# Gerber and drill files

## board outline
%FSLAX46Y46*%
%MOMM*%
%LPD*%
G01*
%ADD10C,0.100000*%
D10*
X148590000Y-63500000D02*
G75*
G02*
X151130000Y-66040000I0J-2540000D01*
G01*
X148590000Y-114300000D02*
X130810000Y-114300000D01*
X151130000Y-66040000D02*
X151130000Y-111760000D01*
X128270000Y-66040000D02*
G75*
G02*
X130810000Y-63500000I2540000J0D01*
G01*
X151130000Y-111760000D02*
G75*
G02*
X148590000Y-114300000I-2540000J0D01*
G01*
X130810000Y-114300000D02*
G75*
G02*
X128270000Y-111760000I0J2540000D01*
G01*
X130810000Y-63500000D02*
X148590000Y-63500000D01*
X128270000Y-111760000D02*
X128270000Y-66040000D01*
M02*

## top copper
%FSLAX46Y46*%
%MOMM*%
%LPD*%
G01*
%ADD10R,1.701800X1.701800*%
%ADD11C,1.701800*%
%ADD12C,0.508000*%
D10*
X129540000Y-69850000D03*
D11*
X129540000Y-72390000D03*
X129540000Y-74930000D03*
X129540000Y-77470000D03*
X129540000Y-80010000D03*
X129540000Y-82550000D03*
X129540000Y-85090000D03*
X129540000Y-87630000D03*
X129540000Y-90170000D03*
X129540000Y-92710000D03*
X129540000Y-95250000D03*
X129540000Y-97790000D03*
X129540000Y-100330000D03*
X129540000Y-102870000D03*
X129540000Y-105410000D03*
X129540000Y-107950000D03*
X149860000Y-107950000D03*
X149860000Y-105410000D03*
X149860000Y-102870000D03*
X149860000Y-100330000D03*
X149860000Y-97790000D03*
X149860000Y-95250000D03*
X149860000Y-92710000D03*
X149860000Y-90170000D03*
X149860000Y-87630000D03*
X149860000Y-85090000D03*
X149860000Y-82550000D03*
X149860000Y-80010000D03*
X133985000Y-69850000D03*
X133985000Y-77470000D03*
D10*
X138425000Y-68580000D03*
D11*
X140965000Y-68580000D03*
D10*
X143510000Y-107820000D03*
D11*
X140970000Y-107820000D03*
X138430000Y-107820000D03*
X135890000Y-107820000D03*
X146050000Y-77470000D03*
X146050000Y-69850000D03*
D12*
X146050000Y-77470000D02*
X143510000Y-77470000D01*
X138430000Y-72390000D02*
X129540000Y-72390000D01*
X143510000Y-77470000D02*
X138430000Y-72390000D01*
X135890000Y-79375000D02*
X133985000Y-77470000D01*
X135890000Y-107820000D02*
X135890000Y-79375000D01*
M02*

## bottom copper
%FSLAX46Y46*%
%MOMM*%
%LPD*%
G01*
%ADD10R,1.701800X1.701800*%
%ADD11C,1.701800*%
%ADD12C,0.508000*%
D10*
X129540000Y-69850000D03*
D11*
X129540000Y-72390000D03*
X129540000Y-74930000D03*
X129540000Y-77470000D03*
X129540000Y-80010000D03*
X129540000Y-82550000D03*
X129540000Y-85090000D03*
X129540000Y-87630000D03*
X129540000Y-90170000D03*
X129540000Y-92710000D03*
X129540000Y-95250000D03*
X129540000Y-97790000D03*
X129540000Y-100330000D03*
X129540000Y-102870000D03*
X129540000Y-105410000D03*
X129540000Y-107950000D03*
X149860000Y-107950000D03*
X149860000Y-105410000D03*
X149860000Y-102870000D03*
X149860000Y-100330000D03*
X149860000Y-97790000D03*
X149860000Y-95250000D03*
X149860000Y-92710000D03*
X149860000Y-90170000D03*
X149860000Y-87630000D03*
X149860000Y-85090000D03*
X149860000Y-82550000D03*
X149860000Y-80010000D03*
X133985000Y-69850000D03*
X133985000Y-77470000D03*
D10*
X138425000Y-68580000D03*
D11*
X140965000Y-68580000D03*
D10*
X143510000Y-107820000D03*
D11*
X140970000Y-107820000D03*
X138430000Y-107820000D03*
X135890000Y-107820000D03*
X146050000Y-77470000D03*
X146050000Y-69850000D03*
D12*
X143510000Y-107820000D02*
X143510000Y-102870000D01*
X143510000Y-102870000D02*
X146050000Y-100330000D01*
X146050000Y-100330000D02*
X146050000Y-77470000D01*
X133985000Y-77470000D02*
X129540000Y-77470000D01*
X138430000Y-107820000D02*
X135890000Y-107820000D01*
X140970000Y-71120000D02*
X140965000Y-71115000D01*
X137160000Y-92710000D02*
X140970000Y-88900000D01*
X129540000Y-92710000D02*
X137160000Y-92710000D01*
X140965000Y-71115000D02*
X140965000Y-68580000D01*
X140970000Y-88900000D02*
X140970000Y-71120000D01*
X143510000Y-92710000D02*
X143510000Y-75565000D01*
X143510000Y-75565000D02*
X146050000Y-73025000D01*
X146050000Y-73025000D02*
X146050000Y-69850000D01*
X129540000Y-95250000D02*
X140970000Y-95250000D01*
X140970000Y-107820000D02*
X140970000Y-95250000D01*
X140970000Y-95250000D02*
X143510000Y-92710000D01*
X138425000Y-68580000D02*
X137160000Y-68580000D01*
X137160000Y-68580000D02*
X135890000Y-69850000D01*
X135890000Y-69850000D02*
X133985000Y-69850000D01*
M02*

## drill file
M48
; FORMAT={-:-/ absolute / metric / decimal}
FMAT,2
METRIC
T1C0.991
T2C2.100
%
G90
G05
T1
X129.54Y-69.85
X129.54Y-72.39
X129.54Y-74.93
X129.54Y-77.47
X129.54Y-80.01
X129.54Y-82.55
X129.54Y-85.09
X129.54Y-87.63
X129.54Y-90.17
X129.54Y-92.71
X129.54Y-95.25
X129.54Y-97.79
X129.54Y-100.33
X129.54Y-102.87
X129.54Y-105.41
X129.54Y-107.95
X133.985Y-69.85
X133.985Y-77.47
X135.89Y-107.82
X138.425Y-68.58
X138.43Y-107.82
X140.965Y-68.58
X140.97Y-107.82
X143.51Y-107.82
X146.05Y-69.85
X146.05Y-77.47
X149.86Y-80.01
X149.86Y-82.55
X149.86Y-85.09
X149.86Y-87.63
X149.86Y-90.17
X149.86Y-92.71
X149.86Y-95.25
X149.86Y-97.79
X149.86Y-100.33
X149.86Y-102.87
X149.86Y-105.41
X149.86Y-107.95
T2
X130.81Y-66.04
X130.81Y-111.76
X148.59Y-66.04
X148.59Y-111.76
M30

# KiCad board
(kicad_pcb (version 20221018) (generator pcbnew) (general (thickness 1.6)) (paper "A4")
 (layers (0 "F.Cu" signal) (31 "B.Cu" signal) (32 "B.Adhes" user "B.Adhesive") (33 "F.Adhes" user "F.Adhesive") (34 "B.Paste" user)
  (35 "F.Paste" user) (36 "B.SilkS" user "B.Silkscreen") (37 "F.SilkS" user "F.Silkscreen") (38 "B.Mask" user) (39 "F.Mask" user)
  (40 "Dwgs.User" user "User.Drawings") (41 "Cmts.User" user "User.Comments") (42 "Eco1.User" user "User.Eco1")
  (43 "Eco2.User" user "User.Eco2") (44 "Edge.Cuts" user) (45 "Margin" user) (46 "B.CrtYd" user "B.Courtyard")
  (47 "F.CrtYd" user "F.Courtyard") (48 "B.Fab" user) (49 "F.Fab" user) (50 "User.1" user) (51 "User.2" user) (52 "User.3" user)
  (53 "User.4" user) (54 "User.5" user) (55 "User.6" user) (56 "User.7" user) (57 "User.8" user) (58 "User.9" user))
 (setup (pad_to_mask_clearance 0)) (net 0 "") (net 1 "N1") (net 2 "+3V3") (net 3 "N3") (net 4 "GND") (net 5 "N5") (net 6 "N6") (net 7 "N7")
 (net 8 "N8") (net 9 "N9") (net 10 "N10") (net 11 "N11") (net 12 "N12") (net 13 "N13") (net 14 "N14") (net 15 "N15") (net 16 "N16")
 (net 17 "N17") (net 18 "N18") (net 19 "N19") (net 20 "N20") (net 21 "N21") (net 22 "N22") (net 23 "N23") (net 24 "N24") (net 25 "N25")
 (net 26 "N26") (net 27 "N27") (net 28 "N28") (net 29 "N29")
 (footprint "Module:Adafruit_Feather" (layer "F.Cu") (at 129.54 69.85)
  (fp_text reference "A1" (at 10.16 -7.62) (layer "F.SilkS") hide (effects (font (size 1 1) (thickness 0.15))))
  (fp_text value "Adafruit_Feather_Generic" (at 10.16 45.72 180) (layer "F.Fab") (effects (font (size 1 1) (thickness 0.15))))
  (pad "1" thru_hole rect (at 0 0 180) (size 1.7018 1.7018) (drill 0.9906) (layers "*.Cu" "*.Mask") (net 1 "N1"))
  (pad "2" thru_hole circle (at 0 2.54 180) (size 1.7018 1.6) (drill 0.9906) (layers "*.Cu" "*.Mask") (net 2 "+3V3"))
  (pad "3" thru_hole circle (at 0 5.08 180) (size 1.7018 1.6) (drill 0.9906) (layers "*.Cu" "*.Mask") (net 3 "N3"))
  (pad "4" thru_hole circle (at 0 7.62 180) (size 1.7018 1.6) (drill 0.9906) (layers "*.Cu" "*.Mask") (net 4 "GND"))
  (pad "5" thru_hole circle (at 0 10.16 180) (size 1.7018 1.6) (drill 0.9906) (layers "*.Cu" "*.Mask") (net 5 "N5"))
  (pad "6" thru_hole circle (at 0 12.7 180) (size 1.7018 1.6) (drill 0.9906) (layers "*.Cu" "*.Mask") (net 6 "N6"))
  (pad "7" thru_hole circle (at 0 15.24 180) (size 1.7018 1.6) (drill 0.9906) (layers "*.Cu" "*.Mask") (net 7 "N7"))
  (pad "8" thru_hole circle (at 0 17.78 180) (size 1.7018 1.6) (drill 0.9906) (layers "*.Cu" "*.Mask") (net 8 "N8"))
  (pad "9" thru_hole circle (at 0 20.32 180) (size 1.7018 1.6) (drill 0.9906) (layers "*.Cu" "*.Mask") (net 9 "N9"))
  (pad "10" thru_hole circle (at 0 22.86 180) (size 1.7018 1.6) (drill 0.9906) (layers "*.Cu" "*.Mask") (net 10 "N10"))
  (pad "11" thru_hole circle (at 0 25.4 180) (size 1.7018 1.6) (drill 0.9906) (layers "*.Cu" "*.Mask") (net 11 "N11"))
  (pad "12" thru_hole circle (at 0 27.94 180) (size 1.7018 1.6) (drill 0.9906) (layers "*.Cu" "*.Mask") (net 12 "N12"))
  (pad "13" thru_hole circle (at 0 30.48 180) (size 1.7018 1.6) (drill 0.9906) (layers "*.Cu" "*.Mask") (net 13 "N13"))
  (pad "14" thru_hole circle (at 0 33.02 180) (size 1.7018 1.6) (drill 0.9906) (layers "*.Cu" "*.Mask") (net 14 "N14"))
  (pad "15" thru_hole circle (at 0 35.56 180) (size 1.7018 1.6) (drill 0.9906) (layers "*.Cu" "*.Mask") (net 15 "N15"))
  (pad "16" thru_hole circle (at 0 38.1 180) (size 1.7018 1.6) (drill 0.9906) (layers "*.Cu" "*.Mask") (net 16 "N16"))
  (pad "17" thru_hole circle (at 20.32 38.1 180) (size 1.7018 1.6) (drill 0.9906) (layers "*.Cu" "*.Mask") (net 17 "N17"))
  (pad "18" thru_hole circle (at 20.32 35.56 180) (size 1.7018 1.6) (drill 0.9906) (layers "*.Cu" "*.Mask") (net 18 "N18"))
  (pad "19" thru_hole circle (at 20.32 33.02 180) (size 1.7018 1.6) (drill 0.9906) (layers "*.Cu" "*.Mask") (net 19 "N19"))
  (pad "20" thru_hole circle (at 20.32 30.48 180) (size 1.7018 1.6) (drill 0.9906) (layers "*.Cu" "*.Mask") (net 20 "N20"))
  (pad "21" thru_hole circle (at 20.32 27.94 180) (size 1.7018 1.6) (drill 0.9906) (layers "*.Cu" "*.Mask") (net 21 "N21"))
  (pad "22" thru_hole circle (at 20.32 25.4 180) (size 1.7018 1.6) (drill 0.9906) (layers "*.Cu" "*.Mask") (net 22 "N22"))
  (pad "23" thru_hole circle (at 20.32 22.86 180) (size 1.7018 1.6) (drill 0.9906) (layers "*.Cu" "*.Mask") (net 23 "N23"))
  (pad "24" thru_hole circle (at 20.32 20.32 180) (size 1.7018 1.6) (drill 0.9906) (layers "*.Cu" "*.Mask") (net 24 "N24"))
  (pad "25" thru_hole circle (at 20.32 17.78 180) (size 1.7018 1.6) (drill 0.9906) (layers "*.Cu" "*.Mask") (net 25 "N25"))
  (pad "26" thru_hole circle (at 20.32 15.24 180) (size 1.7018 1.6) (drill 0.9906) (layers "*.Cu" "*.Mask") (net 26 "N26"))
  (pad "27" thru_hole circle (at 20.32 12.7 180) (size 1.7018 1.6) (drill 0.9906) (layers "*.Cu" "*.Mask") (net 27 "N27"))
  (pad "28" thru_hole circle (at 20.32 10.16 180) (size 1.7018 1.6) (drill 0.9906) (layers "*.Cu" "*.Mask") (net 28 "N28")))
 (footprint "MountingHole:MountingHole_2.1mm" (layer "F.Cu") (at 130.81 111.76)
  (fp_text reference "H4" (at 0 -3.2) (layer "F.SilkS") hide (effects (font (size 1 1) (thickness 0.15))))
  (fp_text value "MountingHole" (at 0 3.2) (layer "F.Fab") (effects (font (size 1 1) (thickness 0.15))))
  (pad "" np_thru_hole circle (at 0 0) (size 2.1 2.1) (drill 2.1) (layers "*.Cu" "*.Mask")))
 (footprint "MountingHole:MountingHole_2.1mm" (layer "F.Cu") (at 148.59 111.76)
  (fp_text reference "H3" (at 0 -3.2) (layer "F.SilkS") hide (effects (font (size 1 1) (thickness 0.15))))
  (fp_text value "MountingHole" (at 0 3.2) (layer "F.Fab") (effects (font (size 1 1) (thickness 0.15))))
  (pad "" np_thru_hole circle (at 0 0) (size 2.1 2.1) (drill 2.1) (layers "*.Cu" "*.Mask")))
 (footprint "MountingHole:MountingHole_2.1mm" (layer "F.Cu") (at 148.59 66.04)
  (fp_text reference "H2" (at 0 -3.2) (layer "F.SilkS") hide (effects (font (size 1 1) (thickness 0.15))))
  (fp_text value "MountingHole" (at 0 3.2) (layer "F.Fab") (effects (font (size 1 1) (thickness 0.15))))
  (pad "" np_thru_hole circle (at 0 0) (size 2.1 2.1) (drill 2.1) (layers "*.Cu" "*.Mask")))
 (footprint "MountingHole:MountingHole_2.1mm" (layer "F.Cu") (at 130.81 66.04)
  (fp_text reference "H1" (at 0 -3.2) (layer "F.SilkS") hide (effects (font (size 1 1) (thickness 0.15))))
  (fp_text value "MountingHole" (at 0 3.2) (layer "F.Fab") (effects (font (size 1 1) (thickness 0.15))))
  (pad "" np_thru_hole circle (at 0 0) (size 2.1 2.1) (drill 2.1) (layers "*.Cu" "*.Mask")))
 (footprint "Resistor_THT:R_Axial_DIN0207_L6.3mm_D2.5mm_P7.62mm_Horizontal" (layer "B.Cu") (at 133.985 69.85 -90)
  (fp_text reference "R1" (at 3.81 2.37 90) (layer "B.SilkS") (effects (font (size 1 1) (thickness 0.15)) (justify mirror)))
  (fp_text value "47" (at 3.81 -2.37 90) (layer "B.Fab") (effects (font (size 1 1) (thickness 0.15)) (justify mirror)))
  (pad "1" thru_hole circle (at 0 0 270) (size 1.7018 1.6) (drill 0.9906) (layers "*.Cu" "*.Mask") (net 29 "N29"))
  (pad "2" thru_hole circle (at 7.62 0 270) (size 1.7018 1.6) (drill 0.9906) (layers "*.Cu" "*.Mask") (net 4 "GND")
   (thermal_bridge_angle 90)))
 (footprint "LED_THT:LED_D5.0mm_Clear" (layer "B.Cu") (at 138.425 68.58)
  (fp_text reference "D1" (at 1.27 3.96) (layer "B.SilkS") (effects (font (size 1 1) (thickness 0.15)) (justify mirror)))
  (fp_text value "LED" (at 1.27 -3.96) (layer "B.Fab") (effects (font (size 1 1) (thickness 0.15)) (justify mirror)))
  (pad "1" thru_hole rect (at 0 0) (size 1.7018 1.7018) (drill 0.9906) (layers "*.Cu" "*.Mask") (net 29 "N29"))
  (pad "2" thru_hole circle (at 2.54 0) (size 1.7018 1.8) (drill 0.9906) (layers "*.Cu" "*.Mask") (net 10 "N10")))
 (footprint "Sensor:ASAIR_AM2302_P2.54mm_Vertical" (layer "B.Cu") (at 143.51 107.82 180)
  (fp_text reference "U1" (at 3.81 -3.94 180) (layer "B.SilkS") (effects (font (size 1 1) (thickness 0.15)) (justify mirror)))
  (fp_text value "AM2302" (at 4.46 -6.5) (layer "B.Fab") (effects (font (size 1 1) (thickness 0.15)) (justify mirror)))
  (pad "1" thru_hole rect (at 0 0 90) (size 1.7018 1.7018) (drill 0.9906) (layers "*.Cu" "*.Mask") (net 2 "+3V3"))
  (pad "2" thru_hole circle (at 2.54 0 90) (size 1.7018 1.7018) (drill 0.9906) (layers "*.Cu" "*.Mask") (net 11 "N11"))
  (pad "3" thru_hole circle (at 5.08 0 90) (size 1.7018 1.7018) (drill 0.9906) (layers "*.Cu" "*.Mask") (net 4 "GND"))
  (pad "4" thru_hole circle (at 7.62 0 90) (size 1.7018 1.7018) (drill 0.9906) (layers "*.Cu" "*.Mask") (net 4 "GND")))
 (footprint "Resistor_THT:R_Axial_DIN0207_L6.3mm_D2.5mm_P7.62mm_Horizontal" (layer "B.Cu") (at 146.05 77.47 90)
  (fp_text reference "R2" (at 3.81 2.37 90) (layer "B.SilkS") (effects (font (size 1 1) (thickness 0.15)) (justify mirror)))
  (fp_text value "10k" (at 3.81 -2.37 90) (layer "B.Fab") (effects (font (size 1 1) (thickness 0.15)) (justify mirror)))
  (pad "1" thru_hole circle (at 0 0 90) (size 1.7018 1.6) (drill 0.9906) (layers "*.Cu" "*.Mask") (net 2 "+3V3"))
  (pad "2" thru_hole circle (at 7.62 0 90) (size 1.7018 1.6) (drill 0.9906) (layers "*.Cu" "*.Mask") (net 11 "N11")
   (thermal_bridge_angle 90)))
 (gr_arc (start 148.59 63.5) (mid 150.386051 64.243949) (end 151.13 66.04) (stroke (width 0.1) (type default)) (layer "Edge.Cuts"))
 (gr_line (start 148.59 114.3) (end 130.81 114.3) (stroke (width 0.1) (type default)) (layer "Edge.Cuts"))
 (gr_line (start 151.13 66.04) (end 151.13 111.76) (stroke (width 0.1) (type default)) (layer "Edge.Cuts"))
 (gr_arc (start 128.27 66.04) (mid 129.013949 64.243949) (end 130.81 63.5) (stroke (width 0.1) (type default)) (layer "Edge.Cuts"))
 (gr_arc (start 151.13 111.76) (mid 150.386051 113.556051) (end 148.59 114.3) (stroke (width 0.1) (type default)) (layer "Edge.Cuts"))
 (gr_arc (start 130.81 114.3) (mid 129.013949 113.556051) (end 128.27 111.76) (stroke (width 0.1) (type default)) (layer "Edge.Cuts"))
 (gr_line (start 130.81 63.5) (end 148.59 63.5) (stroke (width 0.1) (type default)) (layer "Edge.Cuts"))
 (gr_line (start 128.27 111.76) (end 128.27 66.04) (stroke (width 0.1) (type default)) (layer "Edge.Cuts"))
 (segment (start 146.05 77.47) (end 143.51 77.47) (width 0.508) (layer "F.Cu") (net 2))
 (segment (start 138.43 72.39) (end 129.54 72.39) (width 0.508) (layer "F.Cu") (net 2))
 (segment (start 143.51 77.47) (end 138.43 72.39) (width 0.508) (layer "F.Cu") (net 2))
 (segment (start 143.51 107.82) (end 143.51 102.87) (width 0.508) (layer "B.Cu") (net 2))
 (segment (start 143.51 102.87) (end 146.05 100.33) (width 0.508) (layer "B.Cu") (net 2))
 (segment (start 146.05 100.33) (end 146.05 77.47) (width 0.508) (layer "B.Cu") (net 2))
 (segment (start 135.89 79.375) (end 133.985 77.47) (width 0.508) (layer "F.Cu") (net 4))
 (segment (start 135.89 107.82) (end 135.89 79.375) (width 0.508) (layer "F.Cu") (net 4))
 (segment (start 133.985 77.47) (end 129.54 77.47) (width 0.508) (layer "B.Cu") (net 4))
 (segment (start 138.43 107.82) (end 135.89 107.82) (width 0.508) (layer "B.Cu") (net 4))
 (segment (start 140.97 71.12) (end 140.965 71.115) (width 0.508) (layer "B.Cu") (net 10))
 (segment (start 137.16 92.71) (end 140.97 88.9) (width 0.508) (layer "B.Cu") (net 10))
 (segment (start 129.54 92.71) (end 137.16 92.71) (width 0.508) (layer "B.Cu") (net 10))
 (segment (start 140.965 71.115) (end 140.965 68.58) (width 0.508) (layer "B.Cu") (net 10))
 (segment (start 140.97 88.9) (end 140.97 71.12) (width 0.508) (layer "B.Cu") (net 10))
 (segment (start 143.51 92.71) (end 143.51 75.565) (width 0.508) (layer "B.Cu") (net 11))
 (segment (start 143.51 75.565) (end 146.05 73.025) (width 0.508) (layer "B.Cu") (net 11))
 (segment (start 146.05 73.025) (end 146.05 69.85) (width 0.508) (layer "B.Cu") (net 11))
 (segment (start 129.54 95.25) (end 140.97 95.25) (width 0.508) (layer "B.Cu") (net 11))
 (segment (start 140.97 107.82) (end 140.97 95.25) (width 0.508) (layer "B.Cu") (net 11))
 (segment (start 140.97 95.25) (end 143.51 92.71) (width 0.508) (layer "B.Cu") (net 11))
 (segment (start 138.425 68.58) (end 137.16 68.58) (width 0.508) (layer "B.Cu") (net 29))
 (segment (start 137.16 68.58) (end 135.89 69.85) (width 0.508) (layer "B.Cu") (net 29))
 (segment (start 135.89 69.85) (end 133.985 69.85) (width 0.508) (layer "B.Cu") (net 29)))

